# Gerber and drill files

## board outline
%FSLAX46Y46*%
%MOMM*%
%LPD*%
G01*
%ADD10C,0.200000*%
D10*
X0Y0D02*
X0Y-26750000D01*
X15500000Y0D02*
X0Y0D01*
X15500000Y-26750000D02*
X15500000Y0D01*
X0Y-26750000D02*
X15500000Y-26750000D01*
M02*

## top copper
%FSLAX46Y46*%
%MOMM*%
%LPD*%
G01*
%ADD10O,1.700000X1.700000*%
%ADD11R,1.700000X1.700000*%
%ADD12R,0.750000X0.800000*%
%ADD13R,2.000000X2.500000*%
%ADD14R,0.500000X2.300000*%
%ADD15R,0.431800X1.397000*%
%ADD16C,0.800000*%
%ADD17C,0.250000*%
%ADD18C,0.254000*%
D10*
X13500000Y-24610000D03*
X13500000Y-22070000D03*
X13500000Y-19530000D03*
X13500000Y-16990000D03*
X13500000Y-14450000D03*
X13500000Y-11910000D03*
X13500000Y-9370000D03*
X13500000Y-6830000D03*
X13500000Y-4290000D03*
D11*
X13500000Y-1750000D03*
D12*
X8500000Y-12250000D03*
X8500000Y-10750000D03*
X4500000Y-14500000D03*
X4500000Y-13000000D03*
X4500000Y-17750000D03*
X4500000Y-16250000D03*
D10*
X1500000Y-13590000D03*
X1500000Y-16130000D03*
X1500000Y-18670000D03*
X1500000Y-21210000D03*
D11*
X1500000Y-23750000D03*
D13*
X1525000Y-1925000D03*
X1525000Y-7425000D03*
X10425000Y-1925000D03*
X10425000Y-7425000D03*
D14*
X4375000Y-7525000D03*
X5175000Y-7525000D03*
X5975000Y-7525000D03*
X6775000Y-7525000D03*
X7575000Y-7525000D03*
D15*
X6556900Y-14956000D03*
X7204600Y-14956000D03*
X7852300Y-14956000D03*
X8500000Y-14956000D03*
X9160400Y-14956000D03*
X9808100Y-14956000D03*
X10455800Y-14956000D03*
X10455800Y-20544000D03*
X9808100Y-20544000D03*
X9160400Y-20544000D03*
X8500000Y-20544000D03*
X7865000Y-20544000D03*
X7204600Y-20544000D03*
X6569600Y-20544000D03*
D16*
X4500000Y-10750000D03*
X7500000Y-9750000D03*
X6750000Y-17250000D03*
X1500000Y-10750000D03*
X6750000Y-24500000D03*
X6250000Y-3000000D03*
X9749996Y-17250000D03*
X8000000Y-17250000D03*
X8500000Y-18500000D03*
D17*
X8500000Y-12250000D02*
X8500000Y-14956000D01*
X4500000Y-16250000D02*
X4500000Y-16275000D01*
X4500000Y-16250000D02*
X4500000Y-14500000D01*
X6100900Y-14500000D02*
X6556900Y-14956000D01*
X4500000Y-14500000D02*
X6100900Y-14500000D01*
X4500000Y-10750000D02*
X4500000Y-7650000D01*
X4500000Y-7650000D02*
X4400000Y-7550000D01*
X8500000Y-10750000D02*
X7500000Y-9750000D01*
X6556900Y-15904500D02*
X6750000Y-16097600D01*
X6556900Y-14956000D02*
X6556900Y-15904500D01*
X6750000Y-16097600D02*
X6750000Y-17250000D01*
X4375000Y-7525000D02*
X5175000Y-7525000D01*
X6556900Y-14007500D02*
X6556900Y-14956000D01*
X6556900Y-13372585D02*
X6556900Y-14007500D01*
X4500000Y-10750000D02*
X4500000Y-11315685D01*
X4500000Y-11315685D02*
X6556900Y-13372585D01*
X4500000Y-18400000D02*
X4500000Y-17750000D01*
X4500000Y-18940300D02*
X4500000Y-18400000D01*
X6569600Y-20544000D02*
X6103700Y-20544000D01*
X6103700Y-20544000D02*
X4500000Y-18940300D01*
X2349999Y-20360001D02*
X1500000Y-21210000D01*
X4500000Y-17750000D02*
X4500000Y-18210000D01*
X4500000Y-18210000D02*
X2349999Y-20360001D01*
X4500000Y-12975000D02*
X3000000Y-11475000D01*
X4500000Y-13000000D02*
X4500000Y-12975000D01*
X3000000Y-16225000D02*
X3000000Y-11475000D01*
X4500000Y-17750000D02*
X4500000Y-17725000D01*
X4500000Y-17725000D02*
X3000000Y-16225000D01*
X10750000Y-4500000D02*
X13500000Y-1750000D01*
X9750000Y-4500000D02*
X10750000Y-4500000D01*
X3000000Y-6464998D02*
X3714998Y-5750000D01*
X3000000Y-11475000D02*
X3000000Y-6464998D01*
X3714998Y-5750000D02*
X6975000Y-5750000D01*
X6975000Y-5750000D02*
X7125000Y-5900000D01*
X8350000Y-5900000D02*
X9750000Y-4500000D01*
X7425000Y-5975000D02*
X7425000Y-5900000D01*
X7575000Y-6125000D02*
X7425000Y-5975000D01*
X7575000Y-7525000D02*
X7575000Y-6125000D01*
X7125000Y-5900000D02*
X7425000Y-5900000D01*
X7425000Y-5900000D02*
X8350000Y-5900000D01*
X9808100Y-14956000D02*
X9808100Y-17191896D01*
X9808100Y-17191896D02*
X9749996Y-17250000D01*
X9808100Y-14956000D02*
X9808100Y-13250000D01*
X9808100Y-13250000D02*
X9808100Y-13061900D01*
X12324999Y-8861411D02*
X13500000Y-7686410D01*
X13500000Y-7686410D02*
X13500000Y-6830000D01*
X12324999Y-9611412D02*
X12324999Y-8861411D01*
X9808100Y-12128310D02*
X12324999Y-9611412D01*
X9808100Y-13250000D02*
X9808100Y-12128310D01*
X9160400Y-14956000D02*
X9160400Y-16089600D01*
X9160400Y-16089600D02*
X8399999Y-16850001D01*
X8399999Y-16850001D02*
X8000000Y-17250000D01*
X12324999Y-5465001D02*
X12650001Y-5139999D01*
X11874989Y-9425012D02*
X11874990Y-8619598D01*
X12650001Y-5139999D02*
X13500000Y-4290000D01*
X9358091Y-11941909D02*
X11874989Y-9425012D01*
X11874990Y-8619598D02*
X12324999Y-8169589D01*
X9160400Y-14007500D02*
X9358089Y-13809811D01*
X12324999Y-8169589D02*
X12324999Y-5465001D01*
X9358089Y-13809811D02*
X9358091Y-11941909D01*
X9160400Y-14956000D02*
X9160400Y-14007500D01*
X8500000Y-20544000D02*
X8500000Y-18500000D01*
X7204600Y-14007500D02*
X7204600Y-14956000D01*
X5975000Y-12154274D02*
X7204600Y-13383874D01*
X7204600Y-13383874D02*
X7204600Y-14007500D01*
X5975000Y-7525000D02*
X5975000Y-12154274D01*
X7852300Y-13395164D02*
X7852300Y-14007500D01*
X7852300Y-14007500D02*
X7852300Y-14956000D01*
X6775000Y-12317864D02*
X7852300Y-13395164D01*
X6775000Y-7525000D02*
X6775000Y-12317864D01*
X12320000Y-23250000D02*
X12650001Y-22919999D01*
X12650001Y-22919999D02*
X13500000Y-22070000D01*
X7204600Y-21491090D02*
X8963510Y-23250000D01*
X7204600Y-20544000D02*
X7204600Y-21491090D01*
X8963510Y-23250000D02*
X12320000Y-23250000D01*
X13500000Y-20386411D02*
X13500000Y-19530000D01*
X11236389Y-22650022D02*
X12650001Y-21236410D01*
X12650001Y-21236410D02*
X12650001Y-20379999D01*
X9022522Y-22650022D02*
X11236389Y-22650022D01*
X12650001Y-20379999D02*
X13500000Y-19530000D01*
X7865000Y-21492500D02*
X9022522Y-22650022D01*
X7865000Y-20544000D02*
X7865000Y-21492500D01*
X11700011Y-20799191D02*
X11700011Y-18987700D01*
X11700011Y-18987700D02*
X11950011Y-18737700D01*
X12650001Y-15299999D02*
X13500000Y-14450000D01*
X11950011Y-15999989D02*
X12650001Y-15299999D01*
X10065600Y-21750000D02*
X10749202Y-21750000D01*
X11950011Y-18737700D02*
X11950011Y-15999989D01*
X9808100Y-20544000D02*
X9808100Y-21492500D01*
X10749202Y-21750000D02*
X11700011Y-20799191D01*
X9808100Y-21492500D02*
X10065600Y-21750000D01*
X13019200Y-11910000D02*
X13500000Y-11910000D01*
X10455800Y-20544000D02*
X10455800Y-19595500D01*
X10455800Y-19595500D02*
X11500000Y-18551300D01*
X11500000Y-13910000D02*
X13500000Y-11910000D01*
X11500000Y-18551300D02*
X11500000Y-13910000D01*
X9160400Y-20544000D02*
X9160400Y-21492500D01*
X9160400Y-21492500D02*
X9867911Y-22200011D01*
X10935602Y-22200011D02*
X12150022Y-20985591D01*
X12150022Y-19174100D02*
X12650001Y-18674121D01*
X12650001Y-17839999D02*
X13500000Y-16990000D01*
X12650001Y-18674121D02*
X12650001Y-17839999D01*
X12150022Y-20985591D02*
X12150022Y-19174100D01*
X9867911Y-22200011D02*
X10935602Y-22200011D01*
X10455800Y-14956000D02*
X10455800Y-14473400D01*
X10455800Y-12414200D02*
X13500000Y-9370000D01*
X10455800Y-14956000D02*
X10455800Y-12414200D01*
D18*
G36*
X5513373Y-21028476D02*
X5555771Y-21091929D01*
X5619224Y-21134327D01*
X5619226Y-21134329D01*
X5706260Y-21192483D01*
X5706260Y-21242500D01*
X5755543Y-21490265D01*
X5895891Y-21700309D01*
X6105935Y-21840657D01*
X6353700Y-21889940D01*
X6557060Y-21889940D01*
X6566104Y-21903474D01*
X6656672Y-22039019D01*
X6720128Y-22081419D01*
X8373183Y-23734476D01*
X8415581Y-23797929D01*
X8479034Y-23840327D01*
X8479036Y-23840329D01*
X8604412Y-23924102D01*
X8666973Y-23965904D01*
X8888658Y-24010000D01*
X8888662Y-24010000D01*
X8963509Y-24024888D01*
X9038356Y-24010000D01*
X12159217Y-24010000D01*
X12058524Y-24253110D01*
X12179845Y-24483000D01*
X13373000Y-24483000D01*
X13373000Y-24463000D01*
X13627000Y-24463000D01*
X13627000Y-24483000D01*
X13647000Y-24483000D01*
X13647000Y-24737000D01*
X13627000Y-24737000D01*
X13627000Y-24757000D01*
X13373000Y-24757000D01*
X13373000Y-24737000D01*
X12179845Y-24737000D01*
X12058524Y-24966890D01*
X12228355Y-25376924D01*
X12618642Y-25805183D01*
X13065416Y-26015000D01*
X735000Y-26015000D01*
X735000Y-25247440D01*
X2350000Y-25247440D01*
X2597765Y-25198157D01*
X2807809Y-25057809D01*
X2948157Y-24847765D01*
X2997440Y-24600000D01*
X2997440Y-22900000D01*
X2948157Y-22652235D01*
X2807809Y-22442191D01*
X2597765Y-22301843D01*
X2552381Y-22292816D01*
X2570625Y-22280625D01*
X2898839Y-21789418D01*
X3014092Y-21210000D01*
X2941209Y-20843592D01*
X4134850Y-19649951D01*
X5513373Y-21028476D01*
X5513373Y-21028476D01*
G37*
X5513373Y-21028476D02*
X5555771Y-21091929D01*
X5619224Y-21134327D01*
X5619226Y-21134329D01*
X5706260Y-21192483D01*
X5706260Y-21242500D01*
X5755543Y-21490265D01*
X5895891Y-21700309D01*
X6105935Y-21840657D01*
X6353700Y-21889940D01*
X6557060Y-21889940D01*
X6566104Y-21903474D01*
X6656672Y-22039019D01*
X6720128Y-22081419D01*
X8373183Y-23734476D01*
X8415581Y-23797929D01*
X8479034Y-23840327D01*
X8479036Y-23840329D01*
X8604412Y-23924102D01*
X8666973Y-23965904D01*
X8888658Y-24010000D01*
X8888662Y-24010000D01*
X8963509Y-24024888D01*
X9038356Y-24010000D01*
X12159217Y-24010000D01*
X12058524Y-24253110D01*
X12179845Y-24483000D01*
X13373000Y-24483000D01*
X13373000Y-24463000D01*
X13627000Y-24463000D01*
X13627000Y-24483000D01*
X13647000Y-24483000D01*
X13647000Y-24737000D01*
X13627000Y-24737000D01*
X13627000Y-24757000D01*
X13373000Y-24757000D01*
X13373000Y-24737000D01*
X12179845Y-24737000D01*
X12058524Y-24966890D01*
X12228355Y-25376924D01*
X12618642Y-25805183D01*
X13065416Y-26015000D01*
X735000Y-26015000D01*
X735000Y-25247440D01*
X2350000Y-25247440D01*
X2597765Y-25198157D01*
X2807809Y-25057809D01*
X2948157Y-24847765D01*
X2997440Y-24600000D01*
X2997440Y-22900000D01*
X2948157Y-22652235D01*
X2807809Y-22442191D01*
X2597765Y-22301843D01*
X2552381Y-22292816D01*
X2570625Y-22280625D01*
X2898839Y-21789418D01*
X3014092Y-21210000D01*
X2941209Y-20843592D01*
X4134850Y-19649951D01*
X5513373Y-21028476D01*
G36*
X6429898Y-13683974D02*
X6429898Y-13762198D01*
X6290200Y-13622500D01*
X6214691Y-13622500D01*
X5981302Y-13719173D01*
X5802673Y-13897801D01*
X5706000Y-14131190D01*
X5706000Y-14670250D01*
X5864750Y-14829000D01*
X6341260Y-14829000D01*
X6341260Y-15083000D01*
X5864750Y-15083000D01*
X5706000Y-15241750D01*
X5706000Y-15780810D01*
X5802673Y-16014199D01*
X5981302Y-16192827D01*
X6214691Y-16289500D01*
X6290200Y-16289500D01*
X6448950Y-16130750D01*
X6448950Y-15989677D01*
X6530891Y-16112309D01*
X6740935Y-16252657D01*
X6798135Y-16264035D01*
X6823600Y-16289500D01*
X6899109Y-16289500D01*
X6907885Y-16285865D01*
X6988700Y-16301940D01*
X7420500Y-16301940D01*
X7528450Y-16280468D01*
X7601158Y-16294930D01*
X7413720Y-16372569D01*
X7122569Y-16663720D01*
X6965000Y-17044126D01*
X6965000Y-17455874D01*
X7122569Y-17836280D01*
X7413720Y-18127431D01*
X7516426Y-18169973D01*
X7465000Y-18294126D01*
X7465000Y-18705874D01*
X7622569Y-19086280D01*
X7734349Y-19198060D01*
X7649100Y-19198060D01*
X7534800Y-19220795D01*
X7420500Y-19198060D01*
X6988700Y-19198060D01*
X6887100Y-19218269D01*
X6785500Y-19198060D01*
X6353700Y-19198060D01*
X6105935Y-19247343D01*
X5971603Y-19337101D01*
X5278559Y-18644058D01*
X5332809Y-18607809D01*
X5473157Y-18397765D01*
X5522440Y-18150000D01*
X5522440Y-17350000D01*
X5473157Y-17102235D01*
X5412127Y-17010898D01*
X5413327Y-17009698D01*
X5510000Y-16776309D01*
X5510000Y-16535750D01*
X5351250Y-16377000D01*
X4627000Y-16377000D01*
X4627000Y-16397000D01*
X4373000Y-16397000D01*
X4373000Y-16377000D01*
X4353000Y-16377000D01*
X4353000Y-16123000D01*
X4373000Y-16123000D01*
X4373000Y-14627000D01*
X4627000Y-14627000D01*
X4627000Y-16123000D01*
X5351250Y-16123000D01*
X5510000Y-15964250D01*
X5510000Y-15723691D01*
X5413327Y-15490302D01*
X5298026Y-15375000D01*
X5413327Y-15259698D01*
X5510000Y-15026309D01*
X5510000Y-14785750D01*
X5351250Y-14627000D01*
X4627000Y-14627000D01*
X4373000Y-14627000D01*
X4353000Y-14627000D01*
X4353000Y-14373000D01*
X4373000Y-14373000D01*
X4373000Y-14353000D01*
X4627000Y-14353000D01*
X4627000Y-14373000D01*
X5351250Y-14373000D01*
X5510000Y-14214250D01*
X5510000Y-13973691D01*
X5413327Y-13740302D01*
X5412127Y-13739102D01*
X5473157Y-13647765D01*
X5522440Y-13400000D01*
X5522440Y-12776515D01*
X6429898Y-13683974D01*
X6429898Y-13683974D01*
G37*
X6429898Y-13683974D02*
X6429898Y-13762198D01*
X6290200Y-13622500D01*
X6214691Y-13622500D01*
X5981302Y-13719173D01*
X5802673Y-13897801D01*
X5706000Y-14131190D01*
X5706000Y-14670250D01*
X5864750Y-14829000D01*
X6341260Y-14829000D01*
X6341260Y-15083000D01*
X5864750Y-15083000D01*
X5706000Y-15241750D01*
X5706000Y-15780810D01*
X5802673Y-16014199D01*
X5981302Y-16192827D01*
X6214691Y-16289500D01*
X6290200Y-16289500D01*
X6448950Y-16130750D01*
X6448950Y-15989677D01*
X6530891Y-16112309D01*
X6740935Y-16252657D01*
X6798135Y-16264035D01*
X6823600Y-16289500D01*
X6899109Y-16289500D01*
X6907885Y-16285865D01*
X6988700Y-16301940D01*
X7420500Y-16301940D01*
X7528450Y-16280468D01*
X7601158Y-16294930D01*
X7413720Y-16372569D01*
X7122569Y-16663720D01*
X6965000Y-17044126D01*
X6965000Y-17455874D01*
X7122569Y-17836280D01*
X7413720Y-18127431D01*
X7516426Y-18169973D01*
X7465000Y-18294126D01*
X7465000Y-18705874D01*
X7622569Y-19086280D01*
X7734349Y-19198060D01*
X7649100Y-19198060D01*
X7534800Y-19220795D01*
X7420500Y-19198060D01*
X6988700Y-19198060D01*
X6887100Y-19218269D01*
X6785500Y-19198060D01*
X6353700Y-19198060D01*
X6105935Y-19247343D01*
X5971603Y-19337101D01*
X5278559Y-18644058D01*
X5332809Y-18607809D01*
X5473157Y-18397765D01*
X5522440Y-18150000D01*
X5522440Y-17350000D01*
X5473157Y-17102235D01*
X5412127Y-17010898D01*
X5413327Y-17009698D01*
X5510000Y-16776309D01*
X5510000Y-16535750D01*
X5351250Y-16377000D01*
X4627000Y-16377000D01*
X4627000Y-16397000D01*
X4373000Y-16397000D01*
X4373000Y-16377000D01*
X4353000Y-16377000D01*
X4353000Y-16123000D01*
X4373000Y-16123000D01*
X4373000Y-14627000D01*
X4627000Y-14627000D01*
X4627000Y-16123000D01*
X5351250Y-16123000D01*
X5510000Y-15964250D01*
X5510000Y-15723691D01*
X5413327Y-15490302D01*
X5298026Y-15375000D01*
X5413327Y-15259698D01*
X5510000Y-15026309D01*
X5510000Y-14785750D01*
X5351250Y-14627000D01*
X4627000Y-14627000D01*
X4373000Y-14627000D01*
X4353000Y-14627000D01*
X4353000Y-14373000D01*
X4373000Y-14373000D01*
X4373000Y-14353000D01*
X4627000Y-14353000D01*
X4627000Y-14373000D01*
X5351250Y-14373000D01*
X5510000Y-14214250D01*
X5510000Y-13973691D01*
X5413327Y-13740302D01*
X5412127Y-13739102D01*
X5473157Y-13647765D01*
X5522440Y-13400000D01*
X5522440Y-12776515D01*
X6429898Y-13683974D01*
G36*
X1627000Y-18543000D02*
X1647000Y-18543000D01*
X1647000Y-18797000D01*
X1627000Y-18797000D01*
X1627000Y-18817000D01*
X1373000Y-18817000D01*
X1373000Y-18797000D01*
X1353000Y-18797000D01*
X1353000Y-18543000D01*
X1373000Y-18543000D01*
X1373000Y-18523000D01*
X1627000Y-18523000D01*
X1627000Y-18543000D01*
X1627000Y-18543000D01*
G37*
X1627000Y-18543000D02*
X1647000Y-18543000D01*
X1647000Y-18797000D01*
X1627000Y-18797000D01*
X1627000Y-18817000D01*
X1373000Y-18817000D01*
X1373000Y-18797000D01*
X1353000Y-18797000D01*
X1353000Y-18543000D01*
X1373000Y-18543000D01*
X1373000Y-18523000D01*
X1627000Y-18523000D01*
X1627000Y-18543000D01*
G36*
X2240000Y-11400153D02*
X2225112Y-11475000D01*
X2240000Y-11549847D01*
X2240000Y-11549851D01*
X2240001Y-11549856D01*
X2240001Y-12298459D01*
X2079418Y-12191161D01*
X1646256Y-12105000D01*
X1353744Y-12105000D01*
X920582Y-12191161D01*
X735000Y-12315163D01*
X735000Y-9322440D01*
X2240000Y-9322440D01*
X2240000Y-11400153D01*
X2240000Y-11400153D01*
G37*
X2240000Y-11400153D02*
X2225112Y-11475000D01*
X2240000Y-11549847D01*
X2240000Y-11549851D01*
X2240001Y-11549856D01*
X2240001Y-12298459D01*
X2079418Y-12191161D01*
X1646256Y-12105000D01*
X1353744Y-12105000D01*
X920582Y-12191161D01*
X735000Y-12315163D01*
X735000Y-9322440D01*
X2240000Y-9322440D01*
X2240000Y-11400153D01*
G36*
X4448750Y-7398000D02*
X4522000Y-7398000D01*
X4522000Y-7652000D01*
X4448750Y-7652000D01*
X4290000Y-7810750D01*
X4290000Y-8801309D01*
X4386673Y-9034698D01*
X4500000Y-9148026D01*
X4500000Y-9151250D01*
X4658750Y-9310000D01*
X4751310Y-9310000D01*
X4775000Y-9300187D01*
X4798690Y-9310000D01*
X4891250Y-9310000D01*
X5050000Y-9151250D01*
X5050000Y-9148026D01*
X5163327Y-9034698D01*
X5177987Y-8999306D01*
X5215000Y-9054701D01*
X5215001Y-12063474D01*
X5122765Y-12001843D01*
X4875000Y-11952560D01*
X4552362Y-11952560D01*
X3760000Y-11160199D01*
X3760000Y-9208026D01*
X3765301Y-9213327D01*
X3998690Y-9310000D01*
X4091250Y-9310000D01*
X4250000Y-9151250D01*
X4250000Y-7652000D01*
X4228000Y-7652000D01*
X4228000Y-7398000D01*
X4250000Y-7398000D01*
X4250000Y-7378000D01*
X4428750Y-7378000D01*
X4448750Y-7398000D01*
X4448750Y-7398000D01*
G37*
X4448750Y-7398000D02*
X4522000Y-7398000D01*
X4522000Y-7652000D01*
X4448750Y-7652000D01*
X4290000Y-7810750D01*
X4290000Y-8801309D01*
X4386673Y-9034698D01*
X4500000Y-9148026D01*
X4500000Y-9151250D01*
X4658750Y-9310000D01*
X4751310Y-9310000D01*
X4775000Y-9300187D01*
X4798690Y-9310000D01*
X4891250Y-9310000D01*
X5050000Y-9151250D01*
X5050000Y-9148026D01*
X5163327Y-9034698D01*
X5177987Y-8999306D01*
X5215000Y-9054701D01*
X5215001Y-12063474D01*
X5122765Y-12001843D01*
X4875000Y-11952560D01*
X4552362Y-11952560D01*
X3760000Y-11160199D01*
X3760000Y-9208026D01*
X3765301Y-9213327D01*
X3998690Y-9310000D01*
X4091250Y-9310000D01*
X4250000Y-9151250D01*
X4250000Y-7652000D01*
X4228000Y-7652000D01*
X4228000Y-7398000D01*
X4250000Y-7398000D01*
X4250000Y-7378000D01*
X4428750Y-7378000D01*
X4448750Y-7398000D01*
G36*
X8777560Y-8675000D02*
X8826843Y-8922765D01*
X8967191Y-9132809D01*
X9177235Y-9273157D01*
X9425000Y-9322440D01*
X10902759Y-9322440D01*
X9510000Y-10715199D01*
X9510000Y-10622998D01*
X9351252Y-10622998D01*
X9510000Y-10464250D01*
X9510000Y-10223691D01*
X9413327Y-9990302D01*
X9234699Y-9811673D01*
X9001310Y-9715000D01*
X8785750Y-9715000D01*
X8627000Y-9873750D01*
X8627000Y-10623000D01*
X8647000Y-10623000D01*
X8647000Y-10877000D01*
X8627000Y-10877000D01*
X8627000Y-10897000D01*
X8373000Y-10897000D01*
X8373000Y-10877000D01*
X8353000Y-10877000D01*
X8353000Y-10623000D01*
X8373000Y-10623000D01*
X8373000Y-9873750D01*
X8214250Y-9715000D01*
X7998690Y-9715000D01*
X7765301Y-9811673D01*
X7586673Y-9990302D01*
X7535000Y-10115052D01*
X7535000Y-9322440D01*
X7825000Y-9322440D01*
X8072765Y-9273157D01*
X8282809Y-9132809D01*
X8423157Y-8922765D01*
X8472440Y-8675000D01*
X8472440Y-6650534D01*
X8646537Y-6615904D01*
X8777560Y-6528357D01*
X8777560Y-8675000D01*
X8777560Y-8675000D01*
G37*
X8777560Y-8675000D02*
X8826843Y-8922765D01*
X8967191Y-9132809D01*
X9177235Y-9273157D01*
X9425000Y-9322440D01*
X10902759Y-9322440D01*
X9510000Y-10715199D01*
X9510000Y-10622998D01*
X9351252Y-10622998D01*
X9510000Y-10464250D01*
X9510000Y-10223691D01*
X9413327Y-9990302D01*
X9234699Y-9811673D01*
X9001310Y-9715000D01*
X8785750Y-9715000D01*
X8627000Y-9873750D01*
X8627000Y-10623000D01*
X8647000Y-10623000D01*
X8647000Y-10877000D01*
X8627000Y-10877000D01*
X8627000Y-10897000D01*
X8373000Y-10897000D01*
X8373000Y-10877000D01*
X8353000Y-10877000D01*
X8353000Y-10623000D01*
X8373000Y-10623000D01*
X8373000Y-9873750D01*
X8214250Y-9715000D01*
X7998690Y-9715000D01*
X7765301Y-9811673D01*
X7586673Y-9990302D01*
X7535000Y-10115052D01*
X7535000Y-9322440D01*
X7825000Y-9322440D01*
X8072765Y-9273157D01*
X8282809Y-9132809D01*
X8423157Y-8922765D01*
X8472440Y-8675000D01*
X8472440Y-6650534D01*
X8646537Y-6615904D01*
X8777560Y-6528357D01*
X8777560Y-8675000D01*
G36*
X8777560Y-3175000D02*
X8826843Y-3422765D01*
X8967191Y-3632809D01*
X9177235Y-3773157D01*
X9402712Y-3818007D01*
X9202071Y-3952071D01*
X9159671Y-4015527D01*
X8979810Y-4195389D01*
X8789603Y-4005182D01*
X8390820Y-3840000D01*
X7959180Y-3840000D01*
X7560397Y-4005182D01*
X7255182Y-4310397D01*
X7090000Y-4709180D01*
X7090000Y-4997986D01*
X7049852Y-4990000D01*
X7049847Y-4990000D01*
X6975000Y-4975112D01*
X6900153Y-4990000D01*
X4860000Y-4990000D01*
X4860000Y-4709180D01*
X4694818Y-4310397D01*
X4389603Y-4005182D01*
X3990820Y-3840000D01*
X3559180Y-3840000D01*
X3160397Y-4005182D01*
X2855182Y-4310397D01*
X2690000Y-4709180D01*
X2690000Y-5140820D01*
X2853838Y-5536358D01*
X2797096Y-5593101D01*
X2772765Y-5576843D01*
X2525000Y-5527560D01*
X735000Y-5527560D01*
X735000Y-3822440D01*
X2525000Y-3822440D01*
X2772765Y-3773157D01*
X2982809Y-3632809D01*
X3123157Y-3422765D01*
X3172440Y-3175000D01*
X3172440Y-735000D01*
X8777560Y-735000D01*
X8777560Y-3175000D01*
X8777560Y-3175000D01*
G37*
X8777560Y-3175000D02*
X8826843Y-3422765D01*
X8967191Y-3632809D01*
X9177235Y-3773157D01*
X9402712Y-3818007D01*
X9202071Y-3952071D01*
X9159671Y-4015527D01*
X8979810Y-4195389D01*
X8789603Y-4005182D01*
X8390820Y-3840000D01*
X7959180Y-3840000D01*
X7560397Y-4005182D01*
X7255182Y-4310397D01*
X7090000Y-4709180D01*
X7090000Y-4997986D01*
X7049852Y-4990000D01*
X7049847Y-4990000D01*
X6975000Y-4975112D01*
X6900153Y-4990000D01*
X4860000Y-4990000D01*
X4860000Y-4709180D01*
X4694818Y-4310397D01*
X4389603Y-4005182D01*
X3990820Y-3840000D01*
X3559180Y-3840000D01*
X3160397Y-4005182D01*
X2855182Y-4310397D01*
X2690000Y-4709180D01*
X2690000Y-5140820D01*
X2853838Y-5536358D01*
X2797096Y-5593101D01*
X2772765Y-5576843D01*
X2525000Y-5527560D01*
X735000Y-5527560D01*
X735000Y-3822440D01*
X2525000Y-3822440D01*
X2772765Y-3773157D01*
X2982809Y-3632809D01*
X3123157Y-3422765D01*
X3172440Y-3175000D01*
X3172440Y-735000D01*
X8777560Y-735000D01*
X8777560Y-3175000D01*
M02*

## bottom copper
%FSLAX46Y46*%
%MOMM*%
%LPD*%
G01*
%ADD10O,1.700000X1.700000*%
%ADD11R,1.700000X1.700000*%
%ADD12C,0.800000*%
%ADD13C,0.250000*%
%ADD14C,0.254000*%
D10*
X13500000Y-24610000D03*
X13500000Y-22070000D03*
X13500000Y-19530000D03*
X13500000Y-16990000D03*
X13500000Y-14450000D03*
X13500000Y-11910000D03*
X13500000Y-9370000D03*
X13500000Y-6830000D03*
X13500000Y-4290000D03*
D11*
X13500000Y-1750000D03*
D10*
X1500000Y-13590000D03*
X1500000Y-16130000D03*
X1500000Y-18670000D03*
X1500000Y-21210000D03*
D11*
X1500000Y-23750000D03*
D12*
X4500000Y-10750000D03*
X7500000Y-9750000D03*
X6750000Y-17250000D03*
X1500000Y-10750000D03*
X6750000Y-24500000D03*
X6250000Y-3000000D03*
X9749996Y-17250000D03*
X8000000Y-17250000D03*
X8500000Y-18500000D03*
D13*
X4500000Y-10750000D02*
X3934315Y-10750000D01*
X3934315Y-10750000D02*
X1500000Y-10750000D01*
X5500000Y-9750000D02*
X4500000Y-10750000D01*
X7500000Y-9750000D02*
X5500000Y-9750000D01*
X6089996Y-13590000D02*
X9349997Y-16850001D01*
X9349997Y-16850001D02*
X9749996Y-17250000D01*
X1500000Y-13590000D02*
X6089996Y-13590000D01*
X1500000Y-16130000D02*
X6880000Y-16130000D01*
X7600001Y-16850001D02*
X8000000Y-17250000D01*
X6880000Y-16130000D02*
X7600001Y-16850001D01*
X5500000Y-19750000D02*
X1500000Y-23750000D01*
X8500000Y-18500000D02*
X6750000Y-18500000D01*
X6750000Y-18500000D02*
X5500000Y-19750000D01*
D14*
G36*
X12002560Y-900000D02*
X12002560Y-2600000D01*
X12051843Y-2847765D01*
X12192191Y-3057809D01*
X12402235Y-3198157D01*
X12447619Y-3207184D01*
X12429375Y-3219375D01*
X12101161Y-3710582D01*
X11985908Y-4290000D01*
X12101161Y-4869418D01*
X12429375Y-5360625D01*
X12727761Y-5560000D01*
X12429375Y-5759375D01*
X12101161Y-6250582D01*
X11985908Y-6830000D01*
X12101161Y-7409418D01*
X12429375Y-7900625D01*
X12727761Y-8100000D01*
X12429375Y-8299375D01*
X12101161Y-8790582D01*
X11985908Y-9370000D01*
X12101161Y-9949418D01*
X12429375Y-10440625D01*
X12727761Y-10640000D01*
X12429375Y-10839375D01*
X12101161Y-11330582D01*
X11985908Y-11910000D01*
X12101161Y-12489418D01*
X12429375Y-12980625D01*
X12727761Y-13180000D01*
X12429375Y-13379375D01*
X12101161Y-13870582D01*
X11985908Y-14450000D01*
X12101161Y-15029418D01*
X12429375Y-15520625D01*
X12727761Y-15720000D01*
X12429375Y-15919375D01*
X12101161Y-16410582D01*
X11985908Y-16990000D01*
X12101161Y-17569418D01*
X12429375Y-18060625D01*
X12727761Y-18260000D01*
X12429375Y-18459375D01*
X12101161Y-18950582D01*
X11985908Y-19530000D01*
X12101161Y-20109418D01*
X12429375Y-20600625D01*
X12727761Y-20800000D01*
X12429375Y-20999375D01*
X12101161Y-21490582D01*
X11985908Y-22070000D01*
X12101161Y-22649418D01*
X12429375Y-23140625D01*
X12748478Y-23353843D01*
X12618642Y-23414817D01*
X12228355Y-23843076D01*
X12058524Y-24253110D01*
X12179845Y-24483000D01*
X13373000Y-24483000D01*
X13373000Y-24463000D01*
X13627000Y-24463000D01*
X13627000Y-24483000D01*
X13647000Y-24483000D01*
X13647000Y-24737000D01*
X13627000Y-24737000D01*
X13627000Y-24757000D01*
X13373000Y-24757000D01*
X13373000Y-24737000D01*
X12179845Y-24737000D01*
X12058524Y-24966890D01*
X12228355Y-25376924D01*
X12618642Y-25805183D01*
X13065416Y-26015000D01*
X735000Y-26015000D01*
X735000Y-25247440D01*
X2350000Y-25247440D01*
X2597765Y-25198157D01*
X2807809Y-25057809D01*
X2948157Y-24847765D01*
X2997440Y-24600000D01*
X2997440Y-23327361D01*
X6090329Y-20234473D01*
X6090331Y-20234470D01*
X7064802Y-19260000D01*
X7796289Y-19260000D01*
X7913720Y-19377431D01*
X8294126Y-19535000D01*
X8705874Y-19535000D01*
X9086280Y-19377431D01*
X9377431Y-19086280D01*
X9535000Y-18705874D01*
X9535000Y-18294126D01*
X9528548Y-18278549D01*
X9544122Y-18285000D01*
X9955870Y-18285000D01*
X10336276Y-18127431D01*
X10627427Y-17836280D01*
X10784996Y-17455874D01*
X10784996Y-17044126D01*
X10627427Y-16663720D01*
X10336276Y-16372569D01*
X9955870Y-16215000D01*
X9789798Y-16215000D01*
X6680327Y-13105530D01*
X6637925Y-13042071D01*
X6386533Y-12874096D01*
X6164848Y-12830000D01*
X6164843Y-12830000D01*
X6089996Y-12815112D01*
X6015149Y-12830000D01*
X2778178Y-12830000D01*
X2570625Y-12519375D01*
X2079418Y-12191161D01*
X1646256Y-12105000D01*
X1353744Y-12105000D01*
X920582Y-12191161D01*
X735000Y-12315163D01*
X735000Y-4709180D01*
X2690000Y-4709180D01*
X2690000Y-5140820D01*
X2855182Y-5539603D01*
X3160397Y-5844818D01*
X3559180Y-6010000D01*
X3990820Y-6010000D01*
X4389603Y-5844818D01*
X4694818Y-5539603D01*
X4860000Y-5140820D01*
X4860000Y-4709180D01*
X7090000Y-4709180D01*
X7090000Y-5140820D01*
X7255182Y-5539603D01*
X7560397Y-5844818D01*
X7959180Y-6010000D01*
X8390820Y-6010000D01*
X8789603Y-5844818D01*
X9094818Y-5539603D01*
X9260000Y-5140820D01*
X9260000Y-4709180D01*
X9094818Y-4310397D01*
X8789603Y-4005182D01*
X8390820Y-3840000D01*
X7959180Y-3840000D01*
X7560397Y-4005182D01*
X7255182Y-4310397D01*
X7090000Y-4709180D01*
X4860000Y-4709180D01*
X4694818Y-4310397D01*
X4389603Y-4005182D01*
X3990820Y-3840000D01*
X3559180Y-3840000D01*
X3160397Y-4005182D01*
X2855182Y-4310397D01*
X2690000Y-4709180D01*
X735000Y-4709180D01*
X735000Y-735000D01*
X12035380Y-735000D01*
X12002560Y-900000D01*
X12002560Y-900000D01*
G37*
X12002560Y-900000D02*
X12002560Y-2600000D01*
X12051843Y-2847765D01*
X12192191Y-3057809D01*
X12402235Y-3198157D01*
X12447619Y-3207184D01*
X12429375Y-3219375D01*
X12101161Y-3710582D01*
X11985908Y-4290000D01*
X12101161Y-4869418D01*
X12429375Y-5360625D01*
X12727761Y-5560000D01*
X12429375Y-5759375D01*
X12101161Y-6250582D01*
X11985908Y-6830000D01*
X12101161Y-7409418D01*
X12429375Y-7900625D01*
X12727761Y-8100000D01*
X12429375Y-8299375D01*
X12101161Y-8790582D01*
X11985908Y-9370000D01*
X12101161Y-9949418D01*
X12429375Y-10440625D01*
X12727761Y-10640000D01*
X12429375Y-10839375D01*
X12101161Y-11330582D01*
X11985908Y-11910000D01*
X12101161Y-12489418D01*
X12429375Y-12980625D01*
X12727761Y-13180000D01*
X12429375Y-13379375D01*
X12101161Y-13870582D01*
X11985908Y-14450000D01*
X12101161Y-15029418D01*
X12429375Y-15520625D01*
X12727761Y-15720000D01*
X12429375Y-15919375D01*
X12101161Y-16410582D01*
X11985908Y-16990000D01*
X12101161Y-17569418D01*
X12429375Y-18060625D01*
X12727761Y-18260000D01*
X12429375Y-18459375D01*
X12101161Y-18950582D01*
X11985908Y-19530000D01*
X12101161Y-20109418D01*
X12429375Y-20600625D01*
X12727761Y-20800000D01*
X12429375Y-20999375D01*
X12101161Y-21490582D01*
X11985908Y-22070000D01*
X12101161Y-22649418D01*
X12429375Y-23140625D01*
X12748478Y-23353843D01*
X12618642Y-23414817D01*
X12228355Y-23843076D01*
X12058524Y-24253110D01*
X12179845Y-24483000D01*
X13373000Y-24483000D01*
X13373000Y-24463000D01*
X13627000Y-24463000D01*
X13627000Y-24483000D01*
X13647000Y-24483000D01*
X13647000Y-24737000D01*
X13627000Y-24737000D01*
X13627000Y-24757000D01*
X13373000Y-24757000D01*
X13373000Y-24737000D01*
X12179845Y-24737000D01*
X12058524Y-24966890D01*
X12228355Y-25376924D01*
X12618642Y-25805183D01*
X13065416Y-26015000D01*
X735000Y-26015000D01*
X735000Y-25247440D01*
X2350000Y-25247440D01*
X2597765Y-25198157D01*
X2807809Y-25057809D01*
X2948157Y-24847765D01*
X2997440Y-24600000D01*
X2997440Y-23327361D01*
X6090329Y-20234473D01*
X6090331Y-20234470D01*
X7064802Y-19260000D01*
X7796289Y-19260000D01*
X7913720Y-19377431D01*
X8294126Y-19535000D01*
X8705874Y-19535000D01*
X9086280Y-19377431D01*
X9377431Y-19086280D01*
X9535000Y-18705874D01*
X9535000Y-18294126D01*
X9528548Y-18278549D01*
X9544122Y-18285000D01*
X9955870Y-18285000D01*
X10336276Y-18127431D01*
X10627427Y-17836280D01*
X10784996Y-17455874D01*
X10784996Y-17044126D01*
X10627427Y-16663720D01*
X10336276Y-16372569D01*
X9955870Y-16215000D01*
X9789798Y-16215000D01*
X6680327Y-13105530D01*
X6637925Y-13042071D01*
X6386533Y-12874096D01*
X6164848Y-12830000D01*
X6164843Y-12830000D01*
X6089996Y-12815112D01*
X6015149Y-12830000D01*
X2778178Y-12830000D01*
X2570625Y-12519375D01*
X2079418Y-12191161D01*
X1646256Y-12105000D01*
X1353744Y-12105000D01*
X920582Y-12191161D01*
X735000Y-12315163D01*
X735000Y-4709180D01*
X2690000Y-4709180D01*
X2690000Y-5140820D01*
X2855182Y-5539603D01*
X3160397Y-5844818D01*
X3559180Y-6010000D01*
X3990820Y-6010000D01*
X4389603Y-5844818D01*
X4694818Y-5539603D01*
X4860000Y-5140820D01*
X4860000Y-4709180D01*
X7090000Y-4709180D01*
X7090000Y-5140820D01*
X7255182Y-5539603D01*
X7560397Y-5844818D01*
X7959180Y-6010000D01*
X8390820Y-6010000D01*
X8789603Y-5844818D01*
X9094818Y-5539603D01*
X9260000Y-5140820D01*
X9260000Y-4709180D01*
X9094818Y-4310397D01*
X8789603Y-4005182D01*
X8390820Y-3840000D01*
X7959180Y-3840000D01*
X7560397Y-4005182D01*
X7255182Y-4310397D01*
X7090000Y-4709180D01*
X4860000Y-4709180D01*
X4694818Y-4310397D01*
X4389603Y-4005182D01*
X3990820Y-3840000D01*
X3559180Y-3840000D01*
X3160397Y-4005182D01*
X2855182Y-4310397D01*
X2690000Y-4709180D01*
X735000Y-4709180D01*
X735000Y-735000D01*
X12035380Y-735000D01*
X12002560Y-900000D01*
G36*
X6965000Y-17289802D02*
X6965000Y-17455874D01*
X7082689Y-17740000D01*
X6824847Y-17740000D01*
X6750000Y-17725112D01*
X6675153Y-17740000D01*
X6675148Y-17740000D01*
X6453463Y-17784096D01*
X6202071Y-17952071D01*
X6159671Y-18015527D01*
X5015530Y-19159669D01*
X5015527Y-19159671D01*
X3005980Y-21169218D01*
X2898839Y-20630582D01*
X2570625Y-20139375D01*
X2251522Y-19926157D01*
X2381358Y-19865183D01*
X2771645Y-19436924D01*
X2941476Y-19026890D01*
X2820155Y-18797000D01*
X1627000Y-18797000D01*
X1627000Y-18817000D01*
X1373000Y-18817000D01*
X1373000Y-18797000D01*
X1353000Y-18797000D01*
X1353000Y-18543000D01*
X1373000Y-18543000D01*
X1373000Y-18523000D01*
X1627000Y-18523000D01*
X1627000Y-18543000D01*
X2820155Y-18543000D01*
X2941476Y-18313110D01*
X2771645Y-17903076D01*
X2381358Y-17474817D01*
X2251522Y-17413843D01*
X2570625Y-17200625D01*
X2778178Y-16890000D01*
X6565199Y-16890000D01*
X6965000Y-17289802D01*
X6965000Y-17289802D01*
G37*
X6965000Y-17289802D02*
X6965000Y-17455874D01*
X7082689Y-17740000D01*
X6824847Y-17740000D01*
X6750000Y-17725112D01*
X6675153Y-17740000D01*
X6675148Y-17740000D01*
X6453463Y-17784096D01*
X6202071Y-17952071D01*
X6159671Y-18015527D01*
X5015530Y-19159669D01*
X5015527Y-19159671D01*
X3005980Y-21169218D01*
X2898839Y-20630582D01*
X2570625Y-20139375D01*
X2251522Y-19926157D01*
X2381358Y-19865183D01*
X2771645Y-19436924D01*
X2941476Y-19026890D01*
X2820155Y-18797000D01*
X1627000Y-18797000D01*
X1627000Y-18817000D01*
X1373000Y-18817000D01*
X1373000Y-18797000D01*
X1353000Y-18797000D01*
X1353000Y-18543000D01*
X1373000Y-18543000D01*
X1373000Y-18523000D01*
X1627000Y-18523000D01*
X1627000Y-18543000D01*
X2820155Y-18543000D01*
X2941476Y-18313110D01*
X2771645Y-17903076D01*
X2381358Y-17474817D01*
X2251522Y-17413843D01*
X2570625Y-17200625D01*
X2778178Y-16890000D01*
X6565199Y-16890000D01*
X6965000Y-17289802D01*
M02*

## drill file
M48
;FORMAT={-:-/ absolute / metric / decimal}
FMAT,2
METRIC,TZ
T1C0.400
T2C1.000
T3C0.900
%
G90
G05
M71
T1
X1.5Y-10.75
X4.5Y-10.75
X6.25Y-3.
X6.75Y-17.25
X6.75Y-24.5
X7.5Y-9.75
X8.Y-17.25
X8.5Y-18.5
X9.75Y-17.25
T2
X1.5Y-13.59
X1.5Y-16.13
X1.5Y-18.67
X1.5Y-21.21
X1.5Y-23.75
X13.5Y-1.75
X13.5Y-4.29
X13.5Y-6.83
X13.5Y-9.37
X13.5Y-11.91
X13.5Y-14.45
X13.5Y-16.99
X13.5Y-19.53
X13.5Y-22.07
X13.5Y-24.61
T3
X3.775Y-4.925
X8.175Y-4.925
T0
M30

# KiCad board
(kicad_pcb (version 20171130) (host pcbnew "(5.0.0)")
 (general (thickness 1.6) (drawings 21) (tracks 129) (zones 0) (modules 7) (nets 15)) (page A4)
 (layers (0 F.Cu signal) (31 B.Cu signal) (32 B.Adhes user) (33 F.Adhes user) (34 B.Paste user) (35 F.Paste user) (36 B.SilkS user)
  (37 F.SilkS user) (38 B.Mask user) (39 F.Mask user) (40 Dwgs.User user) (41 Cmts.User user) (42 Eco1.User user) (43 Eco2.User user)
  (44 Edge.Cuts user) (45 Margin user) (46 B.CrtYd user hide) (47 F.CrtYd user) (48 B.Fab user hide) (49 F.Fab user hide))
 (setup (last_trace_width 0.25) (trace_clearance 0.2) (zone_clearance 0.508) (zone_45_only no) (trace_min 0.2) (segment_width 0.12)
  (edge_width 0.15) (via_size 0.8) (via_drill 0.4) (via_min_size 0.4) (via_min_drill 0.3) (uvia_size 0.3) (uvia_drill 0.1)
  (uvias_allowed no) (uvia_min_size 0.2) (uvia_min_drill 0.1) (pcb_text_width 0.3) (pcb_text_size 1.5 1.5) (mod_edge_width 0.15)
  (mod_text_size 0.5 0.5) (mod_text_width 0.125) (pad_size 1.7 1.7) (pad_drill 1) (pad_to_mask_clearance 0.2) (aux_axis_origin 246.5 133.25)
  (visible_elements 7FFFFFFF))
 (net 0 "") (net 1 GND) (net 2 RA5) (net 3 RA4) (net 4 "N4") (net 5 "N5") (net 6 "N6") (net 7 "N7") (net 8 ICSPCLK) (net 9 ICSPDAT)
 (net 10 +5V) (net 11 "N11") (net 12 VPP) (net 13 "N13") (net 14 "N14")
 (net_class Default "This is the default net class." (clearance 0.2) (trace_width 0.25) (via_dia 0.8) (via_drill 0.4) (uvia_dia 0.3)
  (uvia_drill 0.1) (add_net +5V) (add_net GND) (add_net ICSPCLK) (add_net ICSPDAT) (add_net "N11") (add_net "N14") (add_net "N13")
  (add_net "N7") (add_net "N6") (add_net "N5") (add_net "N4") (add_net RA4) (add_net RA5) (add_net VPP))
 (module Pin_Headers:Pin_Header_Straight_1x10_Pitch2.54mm (layer B.Cu) (at 260 135 180)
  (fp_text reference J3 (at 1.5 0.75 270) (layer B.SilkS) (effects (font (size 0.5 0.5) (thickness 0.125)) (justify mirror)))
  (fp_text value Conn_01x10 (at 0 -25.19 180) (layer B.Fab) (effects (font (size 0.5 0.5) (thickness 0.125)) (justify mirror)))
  (pad 10 thru_hole oval (at 0 -22.86 180) (size 1.7 1.7) (drill 1) (layers *.Cu *.Mask) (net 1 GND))
  (pad 9 thru_hole oval (at 0 -20.32 180) (size 1.7 1.7) (drill 1) (layers *.Cu *.Mask) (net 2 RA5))
  (pad 8 thru_hole oval (at 0 -17.78 180) (size 1.7 1.7) (drill 1) (layers *.Cu *.Mask) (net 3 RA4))
  (pad 7 thru_hole oval (at 0 -15.24 180) (size 1.7 1.7) (drill 1) (layers *.Cu *.Mask) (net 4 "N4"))
  (pad 6 thru_hole oval (at 0 -12.7 180) (size 1.7 1.7) (drill 1) (layers *.Cu *.Mask) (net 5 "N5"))
  (pad 5 thru_hole oval (at 0 -10.16 180) (size 1.7 1.7) (drill 1) (layers *.Cu *.Mask) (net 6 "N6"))
  (pad 4 thru_hole oval (at 0 -7.62 180) (size 1.7 1.7) (drill 1) (layers *.Cu *.Mask) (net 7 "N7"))
  (pad 3 thru_hole oval (at 0 -5.08 180) (size 1.7 1.7) (drill 1) (layers *.Cu *.Mask) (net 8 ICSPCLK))
  (pad 2 thru_hole oval (at 0 -2.54 180) (size 1.7 1.7) (drill 1) (layers *.Cu *.Mask) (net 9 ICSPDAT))
  (pad 1 thru_hole rect (at 0 0 180) (size 1.7 1.7) (drill 1) (layers *.Cu *.Mask) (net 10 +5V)))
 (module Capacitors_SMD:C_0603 (layer F.Cu) (at 255 144.75 90)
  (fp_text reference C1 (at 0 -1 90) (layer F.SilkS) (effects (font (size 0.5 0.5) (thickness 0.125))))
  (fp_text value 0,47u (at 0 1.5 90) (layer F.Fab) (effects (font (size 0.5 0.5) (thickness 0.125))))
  (pad 1 smd rect (at -0.75 0 90) (size 0.8 0.75) (layers F.Cu F.Paste F.Mask) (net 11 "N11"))
  (pad 2 smd rect (at 0.75 0 90) (size 0.8 0.75) (layers F.Cu F.Paste F.Mask) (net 1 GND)))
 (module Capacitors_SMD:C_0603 (layer F.Cu) (at 251 147 270)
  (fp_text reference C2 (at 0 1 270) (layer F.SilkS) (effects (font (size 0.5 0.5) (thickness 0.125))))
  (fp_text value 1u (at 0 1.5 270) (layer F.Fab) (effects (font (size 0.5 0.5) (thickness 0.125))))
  (pad 2 smd rect (at 0.75 0 270) (size 0.8 0.75) (layers F.Cu F.Paste F.Mask) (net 1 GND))
  (pad 1 smd rect (at -0.75 0 270) (size 0.8 0.75) (layers F.Cu F.Paste F.Mask) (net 10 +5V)))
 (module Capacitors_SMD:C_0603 (layer F.Cu) (at 251 150.25 90)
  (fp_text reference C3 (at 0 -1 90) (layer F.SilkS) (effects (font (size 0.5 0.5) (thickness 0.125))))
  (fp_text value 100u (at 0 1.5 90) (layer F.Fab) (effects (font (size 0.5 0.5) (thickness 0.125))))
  (pad 1 smd rect (at -0.75 0 90) (size 0.8 0.75) (layers F.Cu F.Paste F.Mask) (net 10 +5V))
  (pad 2 smd rect (at 0.75 0 90) (size 0.8 0.75) (layers F.Cu F.Paste F.Mask) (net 1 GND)))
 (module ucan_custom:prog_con (layer F.Cu) (at 248 157 180)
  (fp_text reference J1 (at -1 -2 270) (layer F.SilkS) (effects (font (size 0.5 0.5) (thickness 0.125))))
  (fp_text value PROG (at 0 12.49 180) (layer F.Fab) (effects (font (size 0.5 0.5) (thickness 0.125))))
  (pad 5 thru_hole oval (at 0 10.16 180) (size 1.7 1.7) (drill 1) (layers *.Cu *.Mask) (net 8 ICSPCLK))
  (pad 4 thru_hole oval (at 0 7.62 180) (size 1.7 1.7) (drill 1) (layers *.Cu *.Mask) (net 9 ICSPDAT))
  (pad 3 thru_hole oval (at 0 5.08 180) (size 1.7 1.7) (drill 1) (layers *.Cu *.Mask) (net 1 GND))
  (pad 2 thru_hole oval (at 0 2.54 180) (size 1.7 1.7) (drill 1) (layers *.Cu *.Mask) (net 10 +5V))
  (pad 1 thru_hole rect (at 0 0 180) (size 1.7 1.7) (drill 1) (layers *.Cu *.Mask) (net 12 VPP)))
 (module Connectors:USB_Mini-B (layer F.Cu) (at 252.475 137.975 270)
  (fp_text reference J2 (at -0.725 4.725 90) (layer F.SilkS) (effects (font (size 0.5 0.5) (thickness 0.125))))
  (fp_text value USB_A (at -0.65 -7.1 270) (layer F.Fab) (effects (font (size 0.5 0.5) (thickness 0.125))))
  (pad "" np_thru_hole circle (at 0.2 2.2 270) (size 0.9 0.9) (drill 0.9) (layers *.Cu *.Mask))
  (pad "" np_thru_hole circle (at 0.2 -2.2 270) (size 0.9 0.9) (drill 0.9) (layers *.Cu *.Mask))
  (pad 6 smd rect (at -2.8 4.45 270) (size 2.5 2) (layers F.Cu F.Paste F.Mask))
  (pad 6 smd rect (at 2.7 4.45 270) (size 2.5 2) (layers F.Cu F.Paste F.Mask))
  (pad 6 smd rect (at -2.8 -4.45 270) (size 2.5 2) (layers F.Cu F.Paste F.Mask))
  (pad 6 smd rect (at 2.7 -4.45 270) (size 2.5 2) (layers F.Cu F.Paste F.Mask))
  (pad 5 smd rect (at 2.8 1.6 270) (size 2.3 0.5) (layers F.Cu F.Paste F.Mask) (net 1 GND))
  (pad 4 smd rect (at 2.8 0.8 270) (size 2.3 0.5) (layers F.Cu F.Paste F.Mask) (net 1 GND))
  (pad 3 smd rect (at 2.8 0 270) (size 2.3 0.5) (layers F.Cu F.Paste F.Mask) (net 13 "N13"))
  (pad 2 smd rect (at 2.8 -0.8 270) (size 2.3 0.5) (layers F.Cu F.Paste F.Mask) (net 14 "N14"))
  (pad 1 smd rect (at 2.8 -1.6 270) (size 2.3 0.5) (layers F.Cu F.Paste F.Mask) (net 10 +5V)))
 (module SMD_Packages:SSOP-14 (layer F.Cu) (at 255 151)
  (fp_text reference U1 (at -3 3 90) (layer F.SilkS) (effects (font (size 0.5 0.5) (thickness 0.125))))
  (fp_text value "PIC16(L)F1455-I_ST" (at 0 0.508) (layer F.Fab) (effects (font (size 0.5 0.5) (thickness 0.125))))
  (pad 14 smd rect (at -1.9431 -2.794) (size 0.4318 1.397) (layers F.Cu F.Paste F.Mask) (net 1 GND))
  (pad 13 smd rect (at -1.2954 -2.794) (size 0.4318 1.397) (layers F.Cu F.Paste F.Mask) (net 13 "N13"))
  (pad 12 smd rect (at -0.6477 -2.794) (size 0.4318 1.397) (layers F.Cu F.Paste F.Mask) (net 14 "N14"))
  (pad 11 smd rect (at 0 -2.794) (size 0.4318 1.397) (layers F.Cu F.Paste F.Mask) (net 11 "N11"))
  (pad 10 smd rect (at 0.6604 -2.794) (size 0.4318 1.397) (layers F.Cu F.Paste F.Mask) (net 9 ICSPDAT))
  (pad 9 smd rect (at 1.3081 -2.794) (size 0.4318 1.397) (layers F.Cu F.Paste F.Mask) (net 8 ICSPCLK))
  (pad 8 smd rect (at 1.9558 -2.794) (size 0.4318 1.397) (layers F.Cu F.Paste F.Mask) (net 7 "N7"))
  (pad 7 smd rect (at 1.9558 2.794) (size 0.4318 1.397) (layers F.Cu F.Paste F.Mask) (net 6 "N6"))
  (pad 6 smd rect (at 1.3081 2.794) (size 0.4318 1.397) (layers F.Cu F.Paste F.Mask) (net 5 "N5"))
  (pad 5 smd rect (at 0.6604 2.794) (size 0.4318 1.397) (layers F.Cu F.Paste F.Mask) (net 4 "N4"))
  (pad 4 smd rect (at 0 2.794) (size 0.4318 1.397) (layers F.Cu F.Paste F.Mask) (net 12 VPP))
  (pad 3 smd rect (at -0.635 2.794) (size 0.4318 1.397) (layers F.Cu F.Paste F.Mask) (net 3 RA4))
  (pad 2 smd rect (at -1.2954 2.794) (size 0.4318 1.397) (layers F.Cu F.Paste F.Mask) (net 2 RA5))
  (pad 1 smd rect (at -1.9304 2.794) (size 0.4318 1.397) (layers F.Cu F.Paste F.Mask) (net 10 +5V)))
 (gr_line (start 246.5 133.25) (end 246.5 160) (layer Edge.Cuts) (width 0.2))
 (gr_line (start 262 133.25) (end 246.5 133.25) (layer Edge.Cuts) (width 0.2))
 (gr_line (start 262 160) (end 262 133.25) (layer Edge.Cuts) (width 0.2))
 (gr_line (start 246.5 160) (end 262 160) (layer Edge.Cuts) (width 0.2))
 (segment (start 255 145.5) (end 255 148.206) (width 0.25) (layer F.Cu) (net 11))
 (segment (start 251 149.5) (end 251 149.525) (width 0.25) (layer F.Cu) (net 1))
 (segment (start 251 149.5) (end 251 147.75) (width 0.25) (layer F.Cu) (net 1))
 (segment (start 252.6009 147.75) (end 253.0569 148.206) (width 0.25) (layer F.Cu) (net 1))
 (segment (start 251 147.75) (end 252.6009 147.75) (width 0.25) (layer F.Cu) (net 1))
 (via (at 251 144) (size 0.8) (drill 0.4) (layers F.Cu B.Cu) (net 1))
 (segment (start 251 144) (end 251 140.9) (width 0.25) (layer F.Cu) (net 1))
 (segment (start 251 140.9) (end 250.9 140.8) (width 0.25) (layer F.Cu) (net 1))
 (via (at 254 143) (size 0.8) (drill 0.4) (layers F.Cu B.Cu) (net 1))
 (segment (start 255 144) (end 254 143) (width 0.25) (layer F.Cu) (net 1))
 (segment (start 253.0569 149.1545) (end 253.25 149.3476) (width 0.25) (layer F.Cu) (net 1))
 (segment (start 253.0569 148.206) (end 253.0569 149.1545) (width 0.25) (layer F.Cu) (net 1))
 (segment (start 253.25 149.3476) (end 253.25 150.5) (width 0.25) (layer F.Cu) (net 1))
 (via (at 253.25 150.5) (size 0.8) (drill 0.4) (layers F.Cu B.Cu) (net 1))
 (segment (start 251 144) (end 250.434315 144) (width 0.25) (layer B.Cu) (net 1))
 (segment (start 250.434315 144) (end 248 144) (width 0.25) (layer B.Cu) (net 1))
 (via (at 248 144) (size 0.8) (drill 0.4) (layers F.Cu B.Cu) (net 1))
 (segment (start 252 143) (end 251 144) (width 0.25) (layer B.Cu) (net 1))
 (segment (start 254 143) (end 252 143) (width 0.25) (layer B.Cu) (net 1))
 (via (at 253.25 157.75) (size 0.8) (drill 0.4) (layers F.Cu B.Cu) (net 1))
 (segment (start 250.875 140.775) (end 251.675 140.775) (width 0.25) (layer F.Cu) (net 1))
 (segment (start 253.0569 147.2575) (end 253.0569 148.206) (width 0.25) (layer F.Cu) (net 1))
 (segment (start 253.0569 146.622585) (end 253.0569 147.2575) (width 0.25) (layer F.Cu) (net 1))
 (segment (start 251 144) (end 251 144.565685) (width 0.25) (layer F.Cu) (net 1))
 (segment (start 251 144.565685) (end 253.0569 146.622585) (width 0.25) (layer F.Cu) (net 1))
 (via (at 252.75 136.25) (size 0.8) (drill 0.4) (layers F.Cu B.Cu) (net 1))
 (segment (start 251 151.65) (end 251 151) (width 0.25) (layer F.Cu) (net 10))
 (segment (start 251 152.1903) (end 251 151.65) (width 0.25) (layer F.Cu) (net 10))
 (segment (start 253.0696 153.794) (end 252.6037 153.794) (width 0.25) (layer F.Cu) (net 10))
 (segment (start 252.6037 153.794) (end 251 152.1903) (width 0.25) (layer F.Cu) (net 10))
 (segment (start 248.849999 153.610001) (end 248 154.46) (width 0.25) (layer F.Cu) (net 10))
 (segment (start 251 151) (end 251 151.46) (width 0.25) (layer F.Cu) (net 10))
 (segment (start 251 151.46) (end 248.849999 153.610001) (width 0.25) (layer F.Cu) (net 10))
 (segment (start 251 146.225) (end 249.5 144.725) (width 0.25) (layer F.Cu) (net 10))
 (segment (start 251 146.25) (end 251 146.225) (width 0.25) (layer F.Cu) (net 10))
 (segment (start 249.5 149.475) (end 249.5 144.725) (width 0.25) (layer F.Cu) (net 10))
 (segment (start 251 151) (end 251 150.975) (width 0.25) (layer F.Cu) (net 10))
 (segment (start 251 150.975) (end 249.5 149.475) (width 0.25) (layer F.Cu) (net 10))
 (segment (start 257.25 137.75) (end 260 135) (width 0.25) (layer F.Cu) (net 10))
 (segment (start 256.25 137.75) (end 257.25 137.75) (width 0.25) (layer F.Cu) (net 10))
 (segment (start 249.5 139.714998) (end 250.214998 139) (width 0.25) (layer F.Cu) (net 10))
 (segment (start 249.5 144.725) (end 249.5 139.714998) (width 0.25) (layer F.Cu) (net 10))
 (segment (start 250.214998 139) (end 253.475 139) (width 0.25) (layer F.Cu) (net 10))
 (segment (start 253.475 139) (end 253.625 139.15) (width 0.25) (layer F.Cu) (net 10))
 (segment (start 254.85 139.15) (end 256.25 137.75) (width 0.25) (layer F.Cu) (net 10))
 (segment (start 253.925 139.225) (end 253.925 139.15) (width 0.25) (layer F.Cu) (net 10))
 (segment (start 254.075 139.375) (end 253.925 139.225) (width 0.25) (layer F.Cu) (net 10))
 (segment (start 254.075 140.775) (end 254.075 139.375) (width 0.25) (layer F.Cu) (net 10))
 (segment (start 253.625 139.15) (end 253.925 139.15) (width 0.25) (layer F.Cu) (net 10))
 (segment (start 253.925 139.15) (end 254.85 139.15) (width 0.25) (layer F.Cu) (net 10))
 (segment (start 252.589996 146.84) (end 255.849997 150.100001) (width 0.25) (layer B.Cu) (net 8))
 (via (at 256.249996 150.5) (size 0.8) (drill 0.4) (layers F.Cu B.Cu) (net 8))
 (segment (start 256.3081 148.206) (end 256.3081 150.441896) (width 0.25) (layer F.Cu) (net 8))
 (segment (start 256.3081 150.441896) (end 256.249996 150.5) (width 0.25) (layer F.Cu) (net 8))
 (segment (start 255.849997 150.100001) (end 256.249996 150.5) (width 0.25) (layer B.Cu) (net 8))
 (segment (start 248 146.84) (end 252.589996 146.84) (width 0.25) (layer B.Cu) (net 8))
 (segment (start 256.3081 148.206) (end 256.3081 146.5) (width 0.25) (layer F.Cu) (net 8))
 (segment (start 256.3081 146.5) (end 256.3081 146.3119) (width 0.25) (layer F.Cu) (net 8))
 (segment (start 258.824999 142.111411) (end 260 140.93641) (width 0.25) (layer F.Cu) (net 8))
 (segment (start 260 140.93641) (end 260 140.08) (width 0.25) (layer F.Cu) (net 8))
 (segment (start 258.824999 142.861412) (end 258.824999 142.111411) (width 0.25) (layer F.Cu) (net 8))
 (segment (start 256.3081 145.37831) (end 258.824999 142.861412) (width 0.25) (layer F.Cu) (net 8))
 (segment (start 256.3081 146.5) (end 256.3081 145.37831) (width 0.25) (layer F.Cu) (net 8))
 (segment (start 248 149.38) (end 253.38 149.38) (width 0.25) (layer B.Cu) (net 9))
 (segment (start 255.6604 148.206) (end 255.6604 149.3396) (width 0.25) (layer F.Cu) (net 9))
 (segment (start 255.6604 149.3396) (end 254.899999 150.100001) (width 0.25) (layer F.Cu) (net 9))
 (segment (start 254.100001 150.100001) (end 254.5 150.5) (width 0.25) (layer B.Cu) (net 9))
 (segment (start 253.38 149.38) (end 254.100001 150.100001) (width 0.25) (layer B.Cu) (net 9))
 (segment (start 254.899999 150.100001) (end 254.5 150.5) (width 0.25) (layer F.Cu) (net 9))
 (via (at 254.5 150.5) (size 0.8) (drill 0.4) (layers F.Cu B.Cu) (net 9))
 (segment (start 258.824999 138.715001) (end 259.150001 138.389999) (width 0.25) (layer F.Cu) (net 9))
 (segment (start 258.374989 142.675012) (end 258.37499 141.869598) (width 0.25) (layer F.Cu) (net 9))
 (segment (start 259.150001 138.389999) (end 260 137.54) (width 0.25) (layer F.Cu) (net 9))
 (segment (start 255.858091 145.191909) (end 258.374989 142.675012) (width 0.25) (layer F.Cu) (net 9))
 (segment (start 258.37499 141.869598) (end 258.824999 141.419589) (width 0.25) (layer F.Cu) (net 9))
 (segment (start 255.6604 147.2575) (end 255.858089 147.059811) (width 0.25) (layer F.Cu) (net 9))
 (segment (start 258.824999 141.419589) (end 258.824999 138.715001) (width 0.25) (layer F.Cu) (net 9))
 (segment (start 255.858089 147.059811) (end 255.858091 145.191909) (width 0.25) (layer F.Cu) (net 9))
 (segment (start 255.6604 148.206) (end 255.6604 147.2575) (width 0.25) (layer F.Cu) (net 9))
 (via (at 255 151.75) (size 0.8) (drill 0.4) (layers F.Cu B.Cu) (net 12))
 (segment (start 255 153.794) (end 255 151.75) (width 0.25) (layer F.Cu) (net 12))
 (segment (start 252 153) (end 248 157) (width 0.25) (layer B.Cu) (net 12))
 (segment (start 255 151.75) (end 253.25 151.75) (width 0.25) (layer B.Cu) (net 12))
 (segment (start 253.25 151.75) (end 252 153) (width 0.25) (layer B.Cu) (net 12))
 (segment (start 253.7046 147.2575) (end 253.7046 148.206) (width 0.25) (layer F.Cu) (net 13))
 (segment (start 252.475 145.404274) (end 253.7046 146.633874) (width 0.25) (layer F.Cu) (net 13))
 (segment (start 253.7046 146.633874) (end 253.7046 147.2575) (width 0.25) (layer F.Cu) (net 13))
 (segment (start 252.475 140.775) (end 252.475 145.404274) (width 0.25) (layer F.Cu) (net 13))
 (segment (start 254.3523 146.645164) (end 254.3523 147.2575) (width 0.25) (layer F.Cu) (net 14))
 (segment (start 254.3523 147.2575) (end 254.3523 148.206) (width 0.25) (layer F.Cu) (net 14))
 (segment (start 253.275 145.567864) (end 254.3523 146.645164) (width 0.25) (layer F.Cu) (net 14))
 (segment (start 253.275 140.775) (end 253.275 145.567864) (width 0.25) (layer F.Cu) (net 14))
 (segment (start 258.82 156.5) (end 259.150001 156.169999) (width 0.25) (layer F.Cu) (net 2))
 (segment (start 259.150001 156.169999) (end 260 155.32) (width 0.25) (layer F.Cu) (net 2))
 (segment (start 253.7046 154.74109) (end 255.46351 156.5) (width 0.25) (layer F.Cu) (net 2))
 (segment (start 253.7046 153.794) (end 253.7046 154.74109) (width 0.25) (layer F.Cu) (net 2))
 (segment (start 255.46351 156.5) (end 258.82 156.5) (width 0.25) (layer F.Cu) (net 2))
 (segment (start 260 153.636411) (end 260 152.78) (width 0.25) (layer F.Cu) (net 3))
 (segment (start 257.736389 155.900022) (end 259.150001 154.48641) (width 0.25) (layer F.Cu) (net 3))
 (segment (start 259.150001 154.48641) (end 259.150001 153.629999) (width 0.25) (layer F.Cu) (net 3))
 (segment (start 255.522522 155.900022) (end 257.736389 155.900022) (width 0.25) (layer F.Cu) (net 3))
 (segment (start 259.150001 153.629999) (end 260 152.78) (width 0.25) (layer F.Cu) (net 3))
 (segment (start 254.365 154.7425) (end 255.522522 155.900022) (width 0.25) (layer F.Cu) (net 3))
 (segment (start 254.365 153.794) (end 254.365 154.7425) (width 0.25) (layer F.Cu) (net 3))
 (segment (start 258.200011 154.049191) (end 258.200011 152.2377) (width 0.25) (layer F.Cu) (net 5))
 (segment (start 258.200011 152.2377) (end 258.450011 151.9877) (width 0.25) (layer F.Cu) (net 5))
 (segment (start 259.150001 148.549999) (end 260 147.7) (width 0.25) (layer F.Cu) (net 5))
 (segment (start 258.450011 149.249989) (end 259.150001 148.549999) (width 0.25) (layer F.Cu) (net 5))
 (segment (start 256.5656 155) (end 257.249202 155) (width 0.25) (layer F.Cu) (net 5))
 (segment (start 258.450011 151.9877) (end 258.450011 149.249989) (width 0.25) (layer F.Cu) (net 5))
 (segment (start 256.3081 153.794) (end 256.3081 154.7425) (width 0.25) (layer F.Cu) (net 5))
 (segment (start 257.249202 155) (end 258.200011 154.049191) (width 0.25) (layer F.Cu) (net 5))
 (segment (start 256.3081 154.7425) (end 256.5656 155) (width 0.25) (layer F.Cu) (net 5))
 (segment (start 259.5192 145.16) (end 260 145.16) (width 0.25) (layer F.Cu) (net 6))
 (segment (start 256.9558 153.794) (end 256.9558 152.8455) (width 0.25) (layer F.Cu) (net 6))
 (segment (start 256.9558 152.8455) (end 258 151.8013) (width 0.25) (layer F.Cu) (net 6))
 (segment (start 258 147.16) (end 260 145.16) (width 0.25) (layer F.Cu) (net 6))
 (segment (start 258 151.8013) (end 258 147.16) (width 0.25) (layer F.Cu) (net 6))
 (segment (start 255.6604 153.794) (end 255.6604 154.7425) (width 0.25) (layer F.Cu) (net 4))
 (segment (start 255.6604 154.7425) (end 256.367911 155.450011) (width 0.25) (layer F.Cu) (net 4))
 (segment (start 257.435602 155.450011) (end 258.650022 154.235591) (width 0.25) (layer F.Cu) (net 4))
 (segment (start 258.650022 152.4241) (end 259.150001 151.924121) (width 0.25) (layer F.Cu) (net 4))
 (segment (start 259.150001 151.089999) (end 260 150.24) (width 0.25) (layer F.Cu) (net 4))
 (segment (start 259.150001 151.924121) (end 259.150001 151.089999) (width 0.25) (layer F.Cu) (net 4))
 (segment (start 258.650022 154.235591) (end 258.650022 152.4241) (width 0.25) (layer F.Cu) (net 4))
 (segment (start 256.367911 155.450011) (end 257.435602 155.450011) (width 0.25) (layer F.Cu) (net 4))
 (segment (start 256.9558 148.206) (end 256.9558 147.7234) (width 0.25) (layer F.Cu) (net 7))
 (segment (start 256.9558 145.6642) (end 260 142.62) (width 0.25) (layer F.Cu) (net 7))
 (segment (start 256.9558 148.206) (end 256.9558 145.6642) (width 0.25) (layer F.Cu) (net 7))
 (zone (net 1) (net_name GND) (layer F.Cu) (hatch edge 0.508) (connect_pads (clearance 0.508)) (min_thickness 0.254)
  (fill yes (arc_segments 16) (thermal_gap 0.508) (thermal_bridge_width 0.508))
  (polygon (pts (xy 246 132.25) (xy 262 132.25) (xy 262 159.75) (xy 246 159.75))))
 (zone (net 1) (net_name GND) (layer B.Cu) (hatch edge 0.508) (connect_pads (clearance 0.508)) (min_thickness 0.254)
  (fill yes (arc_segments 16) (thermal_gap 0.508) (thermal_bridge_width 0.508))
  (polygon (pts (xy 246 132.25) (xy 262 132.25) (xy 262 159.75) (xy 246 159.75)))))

